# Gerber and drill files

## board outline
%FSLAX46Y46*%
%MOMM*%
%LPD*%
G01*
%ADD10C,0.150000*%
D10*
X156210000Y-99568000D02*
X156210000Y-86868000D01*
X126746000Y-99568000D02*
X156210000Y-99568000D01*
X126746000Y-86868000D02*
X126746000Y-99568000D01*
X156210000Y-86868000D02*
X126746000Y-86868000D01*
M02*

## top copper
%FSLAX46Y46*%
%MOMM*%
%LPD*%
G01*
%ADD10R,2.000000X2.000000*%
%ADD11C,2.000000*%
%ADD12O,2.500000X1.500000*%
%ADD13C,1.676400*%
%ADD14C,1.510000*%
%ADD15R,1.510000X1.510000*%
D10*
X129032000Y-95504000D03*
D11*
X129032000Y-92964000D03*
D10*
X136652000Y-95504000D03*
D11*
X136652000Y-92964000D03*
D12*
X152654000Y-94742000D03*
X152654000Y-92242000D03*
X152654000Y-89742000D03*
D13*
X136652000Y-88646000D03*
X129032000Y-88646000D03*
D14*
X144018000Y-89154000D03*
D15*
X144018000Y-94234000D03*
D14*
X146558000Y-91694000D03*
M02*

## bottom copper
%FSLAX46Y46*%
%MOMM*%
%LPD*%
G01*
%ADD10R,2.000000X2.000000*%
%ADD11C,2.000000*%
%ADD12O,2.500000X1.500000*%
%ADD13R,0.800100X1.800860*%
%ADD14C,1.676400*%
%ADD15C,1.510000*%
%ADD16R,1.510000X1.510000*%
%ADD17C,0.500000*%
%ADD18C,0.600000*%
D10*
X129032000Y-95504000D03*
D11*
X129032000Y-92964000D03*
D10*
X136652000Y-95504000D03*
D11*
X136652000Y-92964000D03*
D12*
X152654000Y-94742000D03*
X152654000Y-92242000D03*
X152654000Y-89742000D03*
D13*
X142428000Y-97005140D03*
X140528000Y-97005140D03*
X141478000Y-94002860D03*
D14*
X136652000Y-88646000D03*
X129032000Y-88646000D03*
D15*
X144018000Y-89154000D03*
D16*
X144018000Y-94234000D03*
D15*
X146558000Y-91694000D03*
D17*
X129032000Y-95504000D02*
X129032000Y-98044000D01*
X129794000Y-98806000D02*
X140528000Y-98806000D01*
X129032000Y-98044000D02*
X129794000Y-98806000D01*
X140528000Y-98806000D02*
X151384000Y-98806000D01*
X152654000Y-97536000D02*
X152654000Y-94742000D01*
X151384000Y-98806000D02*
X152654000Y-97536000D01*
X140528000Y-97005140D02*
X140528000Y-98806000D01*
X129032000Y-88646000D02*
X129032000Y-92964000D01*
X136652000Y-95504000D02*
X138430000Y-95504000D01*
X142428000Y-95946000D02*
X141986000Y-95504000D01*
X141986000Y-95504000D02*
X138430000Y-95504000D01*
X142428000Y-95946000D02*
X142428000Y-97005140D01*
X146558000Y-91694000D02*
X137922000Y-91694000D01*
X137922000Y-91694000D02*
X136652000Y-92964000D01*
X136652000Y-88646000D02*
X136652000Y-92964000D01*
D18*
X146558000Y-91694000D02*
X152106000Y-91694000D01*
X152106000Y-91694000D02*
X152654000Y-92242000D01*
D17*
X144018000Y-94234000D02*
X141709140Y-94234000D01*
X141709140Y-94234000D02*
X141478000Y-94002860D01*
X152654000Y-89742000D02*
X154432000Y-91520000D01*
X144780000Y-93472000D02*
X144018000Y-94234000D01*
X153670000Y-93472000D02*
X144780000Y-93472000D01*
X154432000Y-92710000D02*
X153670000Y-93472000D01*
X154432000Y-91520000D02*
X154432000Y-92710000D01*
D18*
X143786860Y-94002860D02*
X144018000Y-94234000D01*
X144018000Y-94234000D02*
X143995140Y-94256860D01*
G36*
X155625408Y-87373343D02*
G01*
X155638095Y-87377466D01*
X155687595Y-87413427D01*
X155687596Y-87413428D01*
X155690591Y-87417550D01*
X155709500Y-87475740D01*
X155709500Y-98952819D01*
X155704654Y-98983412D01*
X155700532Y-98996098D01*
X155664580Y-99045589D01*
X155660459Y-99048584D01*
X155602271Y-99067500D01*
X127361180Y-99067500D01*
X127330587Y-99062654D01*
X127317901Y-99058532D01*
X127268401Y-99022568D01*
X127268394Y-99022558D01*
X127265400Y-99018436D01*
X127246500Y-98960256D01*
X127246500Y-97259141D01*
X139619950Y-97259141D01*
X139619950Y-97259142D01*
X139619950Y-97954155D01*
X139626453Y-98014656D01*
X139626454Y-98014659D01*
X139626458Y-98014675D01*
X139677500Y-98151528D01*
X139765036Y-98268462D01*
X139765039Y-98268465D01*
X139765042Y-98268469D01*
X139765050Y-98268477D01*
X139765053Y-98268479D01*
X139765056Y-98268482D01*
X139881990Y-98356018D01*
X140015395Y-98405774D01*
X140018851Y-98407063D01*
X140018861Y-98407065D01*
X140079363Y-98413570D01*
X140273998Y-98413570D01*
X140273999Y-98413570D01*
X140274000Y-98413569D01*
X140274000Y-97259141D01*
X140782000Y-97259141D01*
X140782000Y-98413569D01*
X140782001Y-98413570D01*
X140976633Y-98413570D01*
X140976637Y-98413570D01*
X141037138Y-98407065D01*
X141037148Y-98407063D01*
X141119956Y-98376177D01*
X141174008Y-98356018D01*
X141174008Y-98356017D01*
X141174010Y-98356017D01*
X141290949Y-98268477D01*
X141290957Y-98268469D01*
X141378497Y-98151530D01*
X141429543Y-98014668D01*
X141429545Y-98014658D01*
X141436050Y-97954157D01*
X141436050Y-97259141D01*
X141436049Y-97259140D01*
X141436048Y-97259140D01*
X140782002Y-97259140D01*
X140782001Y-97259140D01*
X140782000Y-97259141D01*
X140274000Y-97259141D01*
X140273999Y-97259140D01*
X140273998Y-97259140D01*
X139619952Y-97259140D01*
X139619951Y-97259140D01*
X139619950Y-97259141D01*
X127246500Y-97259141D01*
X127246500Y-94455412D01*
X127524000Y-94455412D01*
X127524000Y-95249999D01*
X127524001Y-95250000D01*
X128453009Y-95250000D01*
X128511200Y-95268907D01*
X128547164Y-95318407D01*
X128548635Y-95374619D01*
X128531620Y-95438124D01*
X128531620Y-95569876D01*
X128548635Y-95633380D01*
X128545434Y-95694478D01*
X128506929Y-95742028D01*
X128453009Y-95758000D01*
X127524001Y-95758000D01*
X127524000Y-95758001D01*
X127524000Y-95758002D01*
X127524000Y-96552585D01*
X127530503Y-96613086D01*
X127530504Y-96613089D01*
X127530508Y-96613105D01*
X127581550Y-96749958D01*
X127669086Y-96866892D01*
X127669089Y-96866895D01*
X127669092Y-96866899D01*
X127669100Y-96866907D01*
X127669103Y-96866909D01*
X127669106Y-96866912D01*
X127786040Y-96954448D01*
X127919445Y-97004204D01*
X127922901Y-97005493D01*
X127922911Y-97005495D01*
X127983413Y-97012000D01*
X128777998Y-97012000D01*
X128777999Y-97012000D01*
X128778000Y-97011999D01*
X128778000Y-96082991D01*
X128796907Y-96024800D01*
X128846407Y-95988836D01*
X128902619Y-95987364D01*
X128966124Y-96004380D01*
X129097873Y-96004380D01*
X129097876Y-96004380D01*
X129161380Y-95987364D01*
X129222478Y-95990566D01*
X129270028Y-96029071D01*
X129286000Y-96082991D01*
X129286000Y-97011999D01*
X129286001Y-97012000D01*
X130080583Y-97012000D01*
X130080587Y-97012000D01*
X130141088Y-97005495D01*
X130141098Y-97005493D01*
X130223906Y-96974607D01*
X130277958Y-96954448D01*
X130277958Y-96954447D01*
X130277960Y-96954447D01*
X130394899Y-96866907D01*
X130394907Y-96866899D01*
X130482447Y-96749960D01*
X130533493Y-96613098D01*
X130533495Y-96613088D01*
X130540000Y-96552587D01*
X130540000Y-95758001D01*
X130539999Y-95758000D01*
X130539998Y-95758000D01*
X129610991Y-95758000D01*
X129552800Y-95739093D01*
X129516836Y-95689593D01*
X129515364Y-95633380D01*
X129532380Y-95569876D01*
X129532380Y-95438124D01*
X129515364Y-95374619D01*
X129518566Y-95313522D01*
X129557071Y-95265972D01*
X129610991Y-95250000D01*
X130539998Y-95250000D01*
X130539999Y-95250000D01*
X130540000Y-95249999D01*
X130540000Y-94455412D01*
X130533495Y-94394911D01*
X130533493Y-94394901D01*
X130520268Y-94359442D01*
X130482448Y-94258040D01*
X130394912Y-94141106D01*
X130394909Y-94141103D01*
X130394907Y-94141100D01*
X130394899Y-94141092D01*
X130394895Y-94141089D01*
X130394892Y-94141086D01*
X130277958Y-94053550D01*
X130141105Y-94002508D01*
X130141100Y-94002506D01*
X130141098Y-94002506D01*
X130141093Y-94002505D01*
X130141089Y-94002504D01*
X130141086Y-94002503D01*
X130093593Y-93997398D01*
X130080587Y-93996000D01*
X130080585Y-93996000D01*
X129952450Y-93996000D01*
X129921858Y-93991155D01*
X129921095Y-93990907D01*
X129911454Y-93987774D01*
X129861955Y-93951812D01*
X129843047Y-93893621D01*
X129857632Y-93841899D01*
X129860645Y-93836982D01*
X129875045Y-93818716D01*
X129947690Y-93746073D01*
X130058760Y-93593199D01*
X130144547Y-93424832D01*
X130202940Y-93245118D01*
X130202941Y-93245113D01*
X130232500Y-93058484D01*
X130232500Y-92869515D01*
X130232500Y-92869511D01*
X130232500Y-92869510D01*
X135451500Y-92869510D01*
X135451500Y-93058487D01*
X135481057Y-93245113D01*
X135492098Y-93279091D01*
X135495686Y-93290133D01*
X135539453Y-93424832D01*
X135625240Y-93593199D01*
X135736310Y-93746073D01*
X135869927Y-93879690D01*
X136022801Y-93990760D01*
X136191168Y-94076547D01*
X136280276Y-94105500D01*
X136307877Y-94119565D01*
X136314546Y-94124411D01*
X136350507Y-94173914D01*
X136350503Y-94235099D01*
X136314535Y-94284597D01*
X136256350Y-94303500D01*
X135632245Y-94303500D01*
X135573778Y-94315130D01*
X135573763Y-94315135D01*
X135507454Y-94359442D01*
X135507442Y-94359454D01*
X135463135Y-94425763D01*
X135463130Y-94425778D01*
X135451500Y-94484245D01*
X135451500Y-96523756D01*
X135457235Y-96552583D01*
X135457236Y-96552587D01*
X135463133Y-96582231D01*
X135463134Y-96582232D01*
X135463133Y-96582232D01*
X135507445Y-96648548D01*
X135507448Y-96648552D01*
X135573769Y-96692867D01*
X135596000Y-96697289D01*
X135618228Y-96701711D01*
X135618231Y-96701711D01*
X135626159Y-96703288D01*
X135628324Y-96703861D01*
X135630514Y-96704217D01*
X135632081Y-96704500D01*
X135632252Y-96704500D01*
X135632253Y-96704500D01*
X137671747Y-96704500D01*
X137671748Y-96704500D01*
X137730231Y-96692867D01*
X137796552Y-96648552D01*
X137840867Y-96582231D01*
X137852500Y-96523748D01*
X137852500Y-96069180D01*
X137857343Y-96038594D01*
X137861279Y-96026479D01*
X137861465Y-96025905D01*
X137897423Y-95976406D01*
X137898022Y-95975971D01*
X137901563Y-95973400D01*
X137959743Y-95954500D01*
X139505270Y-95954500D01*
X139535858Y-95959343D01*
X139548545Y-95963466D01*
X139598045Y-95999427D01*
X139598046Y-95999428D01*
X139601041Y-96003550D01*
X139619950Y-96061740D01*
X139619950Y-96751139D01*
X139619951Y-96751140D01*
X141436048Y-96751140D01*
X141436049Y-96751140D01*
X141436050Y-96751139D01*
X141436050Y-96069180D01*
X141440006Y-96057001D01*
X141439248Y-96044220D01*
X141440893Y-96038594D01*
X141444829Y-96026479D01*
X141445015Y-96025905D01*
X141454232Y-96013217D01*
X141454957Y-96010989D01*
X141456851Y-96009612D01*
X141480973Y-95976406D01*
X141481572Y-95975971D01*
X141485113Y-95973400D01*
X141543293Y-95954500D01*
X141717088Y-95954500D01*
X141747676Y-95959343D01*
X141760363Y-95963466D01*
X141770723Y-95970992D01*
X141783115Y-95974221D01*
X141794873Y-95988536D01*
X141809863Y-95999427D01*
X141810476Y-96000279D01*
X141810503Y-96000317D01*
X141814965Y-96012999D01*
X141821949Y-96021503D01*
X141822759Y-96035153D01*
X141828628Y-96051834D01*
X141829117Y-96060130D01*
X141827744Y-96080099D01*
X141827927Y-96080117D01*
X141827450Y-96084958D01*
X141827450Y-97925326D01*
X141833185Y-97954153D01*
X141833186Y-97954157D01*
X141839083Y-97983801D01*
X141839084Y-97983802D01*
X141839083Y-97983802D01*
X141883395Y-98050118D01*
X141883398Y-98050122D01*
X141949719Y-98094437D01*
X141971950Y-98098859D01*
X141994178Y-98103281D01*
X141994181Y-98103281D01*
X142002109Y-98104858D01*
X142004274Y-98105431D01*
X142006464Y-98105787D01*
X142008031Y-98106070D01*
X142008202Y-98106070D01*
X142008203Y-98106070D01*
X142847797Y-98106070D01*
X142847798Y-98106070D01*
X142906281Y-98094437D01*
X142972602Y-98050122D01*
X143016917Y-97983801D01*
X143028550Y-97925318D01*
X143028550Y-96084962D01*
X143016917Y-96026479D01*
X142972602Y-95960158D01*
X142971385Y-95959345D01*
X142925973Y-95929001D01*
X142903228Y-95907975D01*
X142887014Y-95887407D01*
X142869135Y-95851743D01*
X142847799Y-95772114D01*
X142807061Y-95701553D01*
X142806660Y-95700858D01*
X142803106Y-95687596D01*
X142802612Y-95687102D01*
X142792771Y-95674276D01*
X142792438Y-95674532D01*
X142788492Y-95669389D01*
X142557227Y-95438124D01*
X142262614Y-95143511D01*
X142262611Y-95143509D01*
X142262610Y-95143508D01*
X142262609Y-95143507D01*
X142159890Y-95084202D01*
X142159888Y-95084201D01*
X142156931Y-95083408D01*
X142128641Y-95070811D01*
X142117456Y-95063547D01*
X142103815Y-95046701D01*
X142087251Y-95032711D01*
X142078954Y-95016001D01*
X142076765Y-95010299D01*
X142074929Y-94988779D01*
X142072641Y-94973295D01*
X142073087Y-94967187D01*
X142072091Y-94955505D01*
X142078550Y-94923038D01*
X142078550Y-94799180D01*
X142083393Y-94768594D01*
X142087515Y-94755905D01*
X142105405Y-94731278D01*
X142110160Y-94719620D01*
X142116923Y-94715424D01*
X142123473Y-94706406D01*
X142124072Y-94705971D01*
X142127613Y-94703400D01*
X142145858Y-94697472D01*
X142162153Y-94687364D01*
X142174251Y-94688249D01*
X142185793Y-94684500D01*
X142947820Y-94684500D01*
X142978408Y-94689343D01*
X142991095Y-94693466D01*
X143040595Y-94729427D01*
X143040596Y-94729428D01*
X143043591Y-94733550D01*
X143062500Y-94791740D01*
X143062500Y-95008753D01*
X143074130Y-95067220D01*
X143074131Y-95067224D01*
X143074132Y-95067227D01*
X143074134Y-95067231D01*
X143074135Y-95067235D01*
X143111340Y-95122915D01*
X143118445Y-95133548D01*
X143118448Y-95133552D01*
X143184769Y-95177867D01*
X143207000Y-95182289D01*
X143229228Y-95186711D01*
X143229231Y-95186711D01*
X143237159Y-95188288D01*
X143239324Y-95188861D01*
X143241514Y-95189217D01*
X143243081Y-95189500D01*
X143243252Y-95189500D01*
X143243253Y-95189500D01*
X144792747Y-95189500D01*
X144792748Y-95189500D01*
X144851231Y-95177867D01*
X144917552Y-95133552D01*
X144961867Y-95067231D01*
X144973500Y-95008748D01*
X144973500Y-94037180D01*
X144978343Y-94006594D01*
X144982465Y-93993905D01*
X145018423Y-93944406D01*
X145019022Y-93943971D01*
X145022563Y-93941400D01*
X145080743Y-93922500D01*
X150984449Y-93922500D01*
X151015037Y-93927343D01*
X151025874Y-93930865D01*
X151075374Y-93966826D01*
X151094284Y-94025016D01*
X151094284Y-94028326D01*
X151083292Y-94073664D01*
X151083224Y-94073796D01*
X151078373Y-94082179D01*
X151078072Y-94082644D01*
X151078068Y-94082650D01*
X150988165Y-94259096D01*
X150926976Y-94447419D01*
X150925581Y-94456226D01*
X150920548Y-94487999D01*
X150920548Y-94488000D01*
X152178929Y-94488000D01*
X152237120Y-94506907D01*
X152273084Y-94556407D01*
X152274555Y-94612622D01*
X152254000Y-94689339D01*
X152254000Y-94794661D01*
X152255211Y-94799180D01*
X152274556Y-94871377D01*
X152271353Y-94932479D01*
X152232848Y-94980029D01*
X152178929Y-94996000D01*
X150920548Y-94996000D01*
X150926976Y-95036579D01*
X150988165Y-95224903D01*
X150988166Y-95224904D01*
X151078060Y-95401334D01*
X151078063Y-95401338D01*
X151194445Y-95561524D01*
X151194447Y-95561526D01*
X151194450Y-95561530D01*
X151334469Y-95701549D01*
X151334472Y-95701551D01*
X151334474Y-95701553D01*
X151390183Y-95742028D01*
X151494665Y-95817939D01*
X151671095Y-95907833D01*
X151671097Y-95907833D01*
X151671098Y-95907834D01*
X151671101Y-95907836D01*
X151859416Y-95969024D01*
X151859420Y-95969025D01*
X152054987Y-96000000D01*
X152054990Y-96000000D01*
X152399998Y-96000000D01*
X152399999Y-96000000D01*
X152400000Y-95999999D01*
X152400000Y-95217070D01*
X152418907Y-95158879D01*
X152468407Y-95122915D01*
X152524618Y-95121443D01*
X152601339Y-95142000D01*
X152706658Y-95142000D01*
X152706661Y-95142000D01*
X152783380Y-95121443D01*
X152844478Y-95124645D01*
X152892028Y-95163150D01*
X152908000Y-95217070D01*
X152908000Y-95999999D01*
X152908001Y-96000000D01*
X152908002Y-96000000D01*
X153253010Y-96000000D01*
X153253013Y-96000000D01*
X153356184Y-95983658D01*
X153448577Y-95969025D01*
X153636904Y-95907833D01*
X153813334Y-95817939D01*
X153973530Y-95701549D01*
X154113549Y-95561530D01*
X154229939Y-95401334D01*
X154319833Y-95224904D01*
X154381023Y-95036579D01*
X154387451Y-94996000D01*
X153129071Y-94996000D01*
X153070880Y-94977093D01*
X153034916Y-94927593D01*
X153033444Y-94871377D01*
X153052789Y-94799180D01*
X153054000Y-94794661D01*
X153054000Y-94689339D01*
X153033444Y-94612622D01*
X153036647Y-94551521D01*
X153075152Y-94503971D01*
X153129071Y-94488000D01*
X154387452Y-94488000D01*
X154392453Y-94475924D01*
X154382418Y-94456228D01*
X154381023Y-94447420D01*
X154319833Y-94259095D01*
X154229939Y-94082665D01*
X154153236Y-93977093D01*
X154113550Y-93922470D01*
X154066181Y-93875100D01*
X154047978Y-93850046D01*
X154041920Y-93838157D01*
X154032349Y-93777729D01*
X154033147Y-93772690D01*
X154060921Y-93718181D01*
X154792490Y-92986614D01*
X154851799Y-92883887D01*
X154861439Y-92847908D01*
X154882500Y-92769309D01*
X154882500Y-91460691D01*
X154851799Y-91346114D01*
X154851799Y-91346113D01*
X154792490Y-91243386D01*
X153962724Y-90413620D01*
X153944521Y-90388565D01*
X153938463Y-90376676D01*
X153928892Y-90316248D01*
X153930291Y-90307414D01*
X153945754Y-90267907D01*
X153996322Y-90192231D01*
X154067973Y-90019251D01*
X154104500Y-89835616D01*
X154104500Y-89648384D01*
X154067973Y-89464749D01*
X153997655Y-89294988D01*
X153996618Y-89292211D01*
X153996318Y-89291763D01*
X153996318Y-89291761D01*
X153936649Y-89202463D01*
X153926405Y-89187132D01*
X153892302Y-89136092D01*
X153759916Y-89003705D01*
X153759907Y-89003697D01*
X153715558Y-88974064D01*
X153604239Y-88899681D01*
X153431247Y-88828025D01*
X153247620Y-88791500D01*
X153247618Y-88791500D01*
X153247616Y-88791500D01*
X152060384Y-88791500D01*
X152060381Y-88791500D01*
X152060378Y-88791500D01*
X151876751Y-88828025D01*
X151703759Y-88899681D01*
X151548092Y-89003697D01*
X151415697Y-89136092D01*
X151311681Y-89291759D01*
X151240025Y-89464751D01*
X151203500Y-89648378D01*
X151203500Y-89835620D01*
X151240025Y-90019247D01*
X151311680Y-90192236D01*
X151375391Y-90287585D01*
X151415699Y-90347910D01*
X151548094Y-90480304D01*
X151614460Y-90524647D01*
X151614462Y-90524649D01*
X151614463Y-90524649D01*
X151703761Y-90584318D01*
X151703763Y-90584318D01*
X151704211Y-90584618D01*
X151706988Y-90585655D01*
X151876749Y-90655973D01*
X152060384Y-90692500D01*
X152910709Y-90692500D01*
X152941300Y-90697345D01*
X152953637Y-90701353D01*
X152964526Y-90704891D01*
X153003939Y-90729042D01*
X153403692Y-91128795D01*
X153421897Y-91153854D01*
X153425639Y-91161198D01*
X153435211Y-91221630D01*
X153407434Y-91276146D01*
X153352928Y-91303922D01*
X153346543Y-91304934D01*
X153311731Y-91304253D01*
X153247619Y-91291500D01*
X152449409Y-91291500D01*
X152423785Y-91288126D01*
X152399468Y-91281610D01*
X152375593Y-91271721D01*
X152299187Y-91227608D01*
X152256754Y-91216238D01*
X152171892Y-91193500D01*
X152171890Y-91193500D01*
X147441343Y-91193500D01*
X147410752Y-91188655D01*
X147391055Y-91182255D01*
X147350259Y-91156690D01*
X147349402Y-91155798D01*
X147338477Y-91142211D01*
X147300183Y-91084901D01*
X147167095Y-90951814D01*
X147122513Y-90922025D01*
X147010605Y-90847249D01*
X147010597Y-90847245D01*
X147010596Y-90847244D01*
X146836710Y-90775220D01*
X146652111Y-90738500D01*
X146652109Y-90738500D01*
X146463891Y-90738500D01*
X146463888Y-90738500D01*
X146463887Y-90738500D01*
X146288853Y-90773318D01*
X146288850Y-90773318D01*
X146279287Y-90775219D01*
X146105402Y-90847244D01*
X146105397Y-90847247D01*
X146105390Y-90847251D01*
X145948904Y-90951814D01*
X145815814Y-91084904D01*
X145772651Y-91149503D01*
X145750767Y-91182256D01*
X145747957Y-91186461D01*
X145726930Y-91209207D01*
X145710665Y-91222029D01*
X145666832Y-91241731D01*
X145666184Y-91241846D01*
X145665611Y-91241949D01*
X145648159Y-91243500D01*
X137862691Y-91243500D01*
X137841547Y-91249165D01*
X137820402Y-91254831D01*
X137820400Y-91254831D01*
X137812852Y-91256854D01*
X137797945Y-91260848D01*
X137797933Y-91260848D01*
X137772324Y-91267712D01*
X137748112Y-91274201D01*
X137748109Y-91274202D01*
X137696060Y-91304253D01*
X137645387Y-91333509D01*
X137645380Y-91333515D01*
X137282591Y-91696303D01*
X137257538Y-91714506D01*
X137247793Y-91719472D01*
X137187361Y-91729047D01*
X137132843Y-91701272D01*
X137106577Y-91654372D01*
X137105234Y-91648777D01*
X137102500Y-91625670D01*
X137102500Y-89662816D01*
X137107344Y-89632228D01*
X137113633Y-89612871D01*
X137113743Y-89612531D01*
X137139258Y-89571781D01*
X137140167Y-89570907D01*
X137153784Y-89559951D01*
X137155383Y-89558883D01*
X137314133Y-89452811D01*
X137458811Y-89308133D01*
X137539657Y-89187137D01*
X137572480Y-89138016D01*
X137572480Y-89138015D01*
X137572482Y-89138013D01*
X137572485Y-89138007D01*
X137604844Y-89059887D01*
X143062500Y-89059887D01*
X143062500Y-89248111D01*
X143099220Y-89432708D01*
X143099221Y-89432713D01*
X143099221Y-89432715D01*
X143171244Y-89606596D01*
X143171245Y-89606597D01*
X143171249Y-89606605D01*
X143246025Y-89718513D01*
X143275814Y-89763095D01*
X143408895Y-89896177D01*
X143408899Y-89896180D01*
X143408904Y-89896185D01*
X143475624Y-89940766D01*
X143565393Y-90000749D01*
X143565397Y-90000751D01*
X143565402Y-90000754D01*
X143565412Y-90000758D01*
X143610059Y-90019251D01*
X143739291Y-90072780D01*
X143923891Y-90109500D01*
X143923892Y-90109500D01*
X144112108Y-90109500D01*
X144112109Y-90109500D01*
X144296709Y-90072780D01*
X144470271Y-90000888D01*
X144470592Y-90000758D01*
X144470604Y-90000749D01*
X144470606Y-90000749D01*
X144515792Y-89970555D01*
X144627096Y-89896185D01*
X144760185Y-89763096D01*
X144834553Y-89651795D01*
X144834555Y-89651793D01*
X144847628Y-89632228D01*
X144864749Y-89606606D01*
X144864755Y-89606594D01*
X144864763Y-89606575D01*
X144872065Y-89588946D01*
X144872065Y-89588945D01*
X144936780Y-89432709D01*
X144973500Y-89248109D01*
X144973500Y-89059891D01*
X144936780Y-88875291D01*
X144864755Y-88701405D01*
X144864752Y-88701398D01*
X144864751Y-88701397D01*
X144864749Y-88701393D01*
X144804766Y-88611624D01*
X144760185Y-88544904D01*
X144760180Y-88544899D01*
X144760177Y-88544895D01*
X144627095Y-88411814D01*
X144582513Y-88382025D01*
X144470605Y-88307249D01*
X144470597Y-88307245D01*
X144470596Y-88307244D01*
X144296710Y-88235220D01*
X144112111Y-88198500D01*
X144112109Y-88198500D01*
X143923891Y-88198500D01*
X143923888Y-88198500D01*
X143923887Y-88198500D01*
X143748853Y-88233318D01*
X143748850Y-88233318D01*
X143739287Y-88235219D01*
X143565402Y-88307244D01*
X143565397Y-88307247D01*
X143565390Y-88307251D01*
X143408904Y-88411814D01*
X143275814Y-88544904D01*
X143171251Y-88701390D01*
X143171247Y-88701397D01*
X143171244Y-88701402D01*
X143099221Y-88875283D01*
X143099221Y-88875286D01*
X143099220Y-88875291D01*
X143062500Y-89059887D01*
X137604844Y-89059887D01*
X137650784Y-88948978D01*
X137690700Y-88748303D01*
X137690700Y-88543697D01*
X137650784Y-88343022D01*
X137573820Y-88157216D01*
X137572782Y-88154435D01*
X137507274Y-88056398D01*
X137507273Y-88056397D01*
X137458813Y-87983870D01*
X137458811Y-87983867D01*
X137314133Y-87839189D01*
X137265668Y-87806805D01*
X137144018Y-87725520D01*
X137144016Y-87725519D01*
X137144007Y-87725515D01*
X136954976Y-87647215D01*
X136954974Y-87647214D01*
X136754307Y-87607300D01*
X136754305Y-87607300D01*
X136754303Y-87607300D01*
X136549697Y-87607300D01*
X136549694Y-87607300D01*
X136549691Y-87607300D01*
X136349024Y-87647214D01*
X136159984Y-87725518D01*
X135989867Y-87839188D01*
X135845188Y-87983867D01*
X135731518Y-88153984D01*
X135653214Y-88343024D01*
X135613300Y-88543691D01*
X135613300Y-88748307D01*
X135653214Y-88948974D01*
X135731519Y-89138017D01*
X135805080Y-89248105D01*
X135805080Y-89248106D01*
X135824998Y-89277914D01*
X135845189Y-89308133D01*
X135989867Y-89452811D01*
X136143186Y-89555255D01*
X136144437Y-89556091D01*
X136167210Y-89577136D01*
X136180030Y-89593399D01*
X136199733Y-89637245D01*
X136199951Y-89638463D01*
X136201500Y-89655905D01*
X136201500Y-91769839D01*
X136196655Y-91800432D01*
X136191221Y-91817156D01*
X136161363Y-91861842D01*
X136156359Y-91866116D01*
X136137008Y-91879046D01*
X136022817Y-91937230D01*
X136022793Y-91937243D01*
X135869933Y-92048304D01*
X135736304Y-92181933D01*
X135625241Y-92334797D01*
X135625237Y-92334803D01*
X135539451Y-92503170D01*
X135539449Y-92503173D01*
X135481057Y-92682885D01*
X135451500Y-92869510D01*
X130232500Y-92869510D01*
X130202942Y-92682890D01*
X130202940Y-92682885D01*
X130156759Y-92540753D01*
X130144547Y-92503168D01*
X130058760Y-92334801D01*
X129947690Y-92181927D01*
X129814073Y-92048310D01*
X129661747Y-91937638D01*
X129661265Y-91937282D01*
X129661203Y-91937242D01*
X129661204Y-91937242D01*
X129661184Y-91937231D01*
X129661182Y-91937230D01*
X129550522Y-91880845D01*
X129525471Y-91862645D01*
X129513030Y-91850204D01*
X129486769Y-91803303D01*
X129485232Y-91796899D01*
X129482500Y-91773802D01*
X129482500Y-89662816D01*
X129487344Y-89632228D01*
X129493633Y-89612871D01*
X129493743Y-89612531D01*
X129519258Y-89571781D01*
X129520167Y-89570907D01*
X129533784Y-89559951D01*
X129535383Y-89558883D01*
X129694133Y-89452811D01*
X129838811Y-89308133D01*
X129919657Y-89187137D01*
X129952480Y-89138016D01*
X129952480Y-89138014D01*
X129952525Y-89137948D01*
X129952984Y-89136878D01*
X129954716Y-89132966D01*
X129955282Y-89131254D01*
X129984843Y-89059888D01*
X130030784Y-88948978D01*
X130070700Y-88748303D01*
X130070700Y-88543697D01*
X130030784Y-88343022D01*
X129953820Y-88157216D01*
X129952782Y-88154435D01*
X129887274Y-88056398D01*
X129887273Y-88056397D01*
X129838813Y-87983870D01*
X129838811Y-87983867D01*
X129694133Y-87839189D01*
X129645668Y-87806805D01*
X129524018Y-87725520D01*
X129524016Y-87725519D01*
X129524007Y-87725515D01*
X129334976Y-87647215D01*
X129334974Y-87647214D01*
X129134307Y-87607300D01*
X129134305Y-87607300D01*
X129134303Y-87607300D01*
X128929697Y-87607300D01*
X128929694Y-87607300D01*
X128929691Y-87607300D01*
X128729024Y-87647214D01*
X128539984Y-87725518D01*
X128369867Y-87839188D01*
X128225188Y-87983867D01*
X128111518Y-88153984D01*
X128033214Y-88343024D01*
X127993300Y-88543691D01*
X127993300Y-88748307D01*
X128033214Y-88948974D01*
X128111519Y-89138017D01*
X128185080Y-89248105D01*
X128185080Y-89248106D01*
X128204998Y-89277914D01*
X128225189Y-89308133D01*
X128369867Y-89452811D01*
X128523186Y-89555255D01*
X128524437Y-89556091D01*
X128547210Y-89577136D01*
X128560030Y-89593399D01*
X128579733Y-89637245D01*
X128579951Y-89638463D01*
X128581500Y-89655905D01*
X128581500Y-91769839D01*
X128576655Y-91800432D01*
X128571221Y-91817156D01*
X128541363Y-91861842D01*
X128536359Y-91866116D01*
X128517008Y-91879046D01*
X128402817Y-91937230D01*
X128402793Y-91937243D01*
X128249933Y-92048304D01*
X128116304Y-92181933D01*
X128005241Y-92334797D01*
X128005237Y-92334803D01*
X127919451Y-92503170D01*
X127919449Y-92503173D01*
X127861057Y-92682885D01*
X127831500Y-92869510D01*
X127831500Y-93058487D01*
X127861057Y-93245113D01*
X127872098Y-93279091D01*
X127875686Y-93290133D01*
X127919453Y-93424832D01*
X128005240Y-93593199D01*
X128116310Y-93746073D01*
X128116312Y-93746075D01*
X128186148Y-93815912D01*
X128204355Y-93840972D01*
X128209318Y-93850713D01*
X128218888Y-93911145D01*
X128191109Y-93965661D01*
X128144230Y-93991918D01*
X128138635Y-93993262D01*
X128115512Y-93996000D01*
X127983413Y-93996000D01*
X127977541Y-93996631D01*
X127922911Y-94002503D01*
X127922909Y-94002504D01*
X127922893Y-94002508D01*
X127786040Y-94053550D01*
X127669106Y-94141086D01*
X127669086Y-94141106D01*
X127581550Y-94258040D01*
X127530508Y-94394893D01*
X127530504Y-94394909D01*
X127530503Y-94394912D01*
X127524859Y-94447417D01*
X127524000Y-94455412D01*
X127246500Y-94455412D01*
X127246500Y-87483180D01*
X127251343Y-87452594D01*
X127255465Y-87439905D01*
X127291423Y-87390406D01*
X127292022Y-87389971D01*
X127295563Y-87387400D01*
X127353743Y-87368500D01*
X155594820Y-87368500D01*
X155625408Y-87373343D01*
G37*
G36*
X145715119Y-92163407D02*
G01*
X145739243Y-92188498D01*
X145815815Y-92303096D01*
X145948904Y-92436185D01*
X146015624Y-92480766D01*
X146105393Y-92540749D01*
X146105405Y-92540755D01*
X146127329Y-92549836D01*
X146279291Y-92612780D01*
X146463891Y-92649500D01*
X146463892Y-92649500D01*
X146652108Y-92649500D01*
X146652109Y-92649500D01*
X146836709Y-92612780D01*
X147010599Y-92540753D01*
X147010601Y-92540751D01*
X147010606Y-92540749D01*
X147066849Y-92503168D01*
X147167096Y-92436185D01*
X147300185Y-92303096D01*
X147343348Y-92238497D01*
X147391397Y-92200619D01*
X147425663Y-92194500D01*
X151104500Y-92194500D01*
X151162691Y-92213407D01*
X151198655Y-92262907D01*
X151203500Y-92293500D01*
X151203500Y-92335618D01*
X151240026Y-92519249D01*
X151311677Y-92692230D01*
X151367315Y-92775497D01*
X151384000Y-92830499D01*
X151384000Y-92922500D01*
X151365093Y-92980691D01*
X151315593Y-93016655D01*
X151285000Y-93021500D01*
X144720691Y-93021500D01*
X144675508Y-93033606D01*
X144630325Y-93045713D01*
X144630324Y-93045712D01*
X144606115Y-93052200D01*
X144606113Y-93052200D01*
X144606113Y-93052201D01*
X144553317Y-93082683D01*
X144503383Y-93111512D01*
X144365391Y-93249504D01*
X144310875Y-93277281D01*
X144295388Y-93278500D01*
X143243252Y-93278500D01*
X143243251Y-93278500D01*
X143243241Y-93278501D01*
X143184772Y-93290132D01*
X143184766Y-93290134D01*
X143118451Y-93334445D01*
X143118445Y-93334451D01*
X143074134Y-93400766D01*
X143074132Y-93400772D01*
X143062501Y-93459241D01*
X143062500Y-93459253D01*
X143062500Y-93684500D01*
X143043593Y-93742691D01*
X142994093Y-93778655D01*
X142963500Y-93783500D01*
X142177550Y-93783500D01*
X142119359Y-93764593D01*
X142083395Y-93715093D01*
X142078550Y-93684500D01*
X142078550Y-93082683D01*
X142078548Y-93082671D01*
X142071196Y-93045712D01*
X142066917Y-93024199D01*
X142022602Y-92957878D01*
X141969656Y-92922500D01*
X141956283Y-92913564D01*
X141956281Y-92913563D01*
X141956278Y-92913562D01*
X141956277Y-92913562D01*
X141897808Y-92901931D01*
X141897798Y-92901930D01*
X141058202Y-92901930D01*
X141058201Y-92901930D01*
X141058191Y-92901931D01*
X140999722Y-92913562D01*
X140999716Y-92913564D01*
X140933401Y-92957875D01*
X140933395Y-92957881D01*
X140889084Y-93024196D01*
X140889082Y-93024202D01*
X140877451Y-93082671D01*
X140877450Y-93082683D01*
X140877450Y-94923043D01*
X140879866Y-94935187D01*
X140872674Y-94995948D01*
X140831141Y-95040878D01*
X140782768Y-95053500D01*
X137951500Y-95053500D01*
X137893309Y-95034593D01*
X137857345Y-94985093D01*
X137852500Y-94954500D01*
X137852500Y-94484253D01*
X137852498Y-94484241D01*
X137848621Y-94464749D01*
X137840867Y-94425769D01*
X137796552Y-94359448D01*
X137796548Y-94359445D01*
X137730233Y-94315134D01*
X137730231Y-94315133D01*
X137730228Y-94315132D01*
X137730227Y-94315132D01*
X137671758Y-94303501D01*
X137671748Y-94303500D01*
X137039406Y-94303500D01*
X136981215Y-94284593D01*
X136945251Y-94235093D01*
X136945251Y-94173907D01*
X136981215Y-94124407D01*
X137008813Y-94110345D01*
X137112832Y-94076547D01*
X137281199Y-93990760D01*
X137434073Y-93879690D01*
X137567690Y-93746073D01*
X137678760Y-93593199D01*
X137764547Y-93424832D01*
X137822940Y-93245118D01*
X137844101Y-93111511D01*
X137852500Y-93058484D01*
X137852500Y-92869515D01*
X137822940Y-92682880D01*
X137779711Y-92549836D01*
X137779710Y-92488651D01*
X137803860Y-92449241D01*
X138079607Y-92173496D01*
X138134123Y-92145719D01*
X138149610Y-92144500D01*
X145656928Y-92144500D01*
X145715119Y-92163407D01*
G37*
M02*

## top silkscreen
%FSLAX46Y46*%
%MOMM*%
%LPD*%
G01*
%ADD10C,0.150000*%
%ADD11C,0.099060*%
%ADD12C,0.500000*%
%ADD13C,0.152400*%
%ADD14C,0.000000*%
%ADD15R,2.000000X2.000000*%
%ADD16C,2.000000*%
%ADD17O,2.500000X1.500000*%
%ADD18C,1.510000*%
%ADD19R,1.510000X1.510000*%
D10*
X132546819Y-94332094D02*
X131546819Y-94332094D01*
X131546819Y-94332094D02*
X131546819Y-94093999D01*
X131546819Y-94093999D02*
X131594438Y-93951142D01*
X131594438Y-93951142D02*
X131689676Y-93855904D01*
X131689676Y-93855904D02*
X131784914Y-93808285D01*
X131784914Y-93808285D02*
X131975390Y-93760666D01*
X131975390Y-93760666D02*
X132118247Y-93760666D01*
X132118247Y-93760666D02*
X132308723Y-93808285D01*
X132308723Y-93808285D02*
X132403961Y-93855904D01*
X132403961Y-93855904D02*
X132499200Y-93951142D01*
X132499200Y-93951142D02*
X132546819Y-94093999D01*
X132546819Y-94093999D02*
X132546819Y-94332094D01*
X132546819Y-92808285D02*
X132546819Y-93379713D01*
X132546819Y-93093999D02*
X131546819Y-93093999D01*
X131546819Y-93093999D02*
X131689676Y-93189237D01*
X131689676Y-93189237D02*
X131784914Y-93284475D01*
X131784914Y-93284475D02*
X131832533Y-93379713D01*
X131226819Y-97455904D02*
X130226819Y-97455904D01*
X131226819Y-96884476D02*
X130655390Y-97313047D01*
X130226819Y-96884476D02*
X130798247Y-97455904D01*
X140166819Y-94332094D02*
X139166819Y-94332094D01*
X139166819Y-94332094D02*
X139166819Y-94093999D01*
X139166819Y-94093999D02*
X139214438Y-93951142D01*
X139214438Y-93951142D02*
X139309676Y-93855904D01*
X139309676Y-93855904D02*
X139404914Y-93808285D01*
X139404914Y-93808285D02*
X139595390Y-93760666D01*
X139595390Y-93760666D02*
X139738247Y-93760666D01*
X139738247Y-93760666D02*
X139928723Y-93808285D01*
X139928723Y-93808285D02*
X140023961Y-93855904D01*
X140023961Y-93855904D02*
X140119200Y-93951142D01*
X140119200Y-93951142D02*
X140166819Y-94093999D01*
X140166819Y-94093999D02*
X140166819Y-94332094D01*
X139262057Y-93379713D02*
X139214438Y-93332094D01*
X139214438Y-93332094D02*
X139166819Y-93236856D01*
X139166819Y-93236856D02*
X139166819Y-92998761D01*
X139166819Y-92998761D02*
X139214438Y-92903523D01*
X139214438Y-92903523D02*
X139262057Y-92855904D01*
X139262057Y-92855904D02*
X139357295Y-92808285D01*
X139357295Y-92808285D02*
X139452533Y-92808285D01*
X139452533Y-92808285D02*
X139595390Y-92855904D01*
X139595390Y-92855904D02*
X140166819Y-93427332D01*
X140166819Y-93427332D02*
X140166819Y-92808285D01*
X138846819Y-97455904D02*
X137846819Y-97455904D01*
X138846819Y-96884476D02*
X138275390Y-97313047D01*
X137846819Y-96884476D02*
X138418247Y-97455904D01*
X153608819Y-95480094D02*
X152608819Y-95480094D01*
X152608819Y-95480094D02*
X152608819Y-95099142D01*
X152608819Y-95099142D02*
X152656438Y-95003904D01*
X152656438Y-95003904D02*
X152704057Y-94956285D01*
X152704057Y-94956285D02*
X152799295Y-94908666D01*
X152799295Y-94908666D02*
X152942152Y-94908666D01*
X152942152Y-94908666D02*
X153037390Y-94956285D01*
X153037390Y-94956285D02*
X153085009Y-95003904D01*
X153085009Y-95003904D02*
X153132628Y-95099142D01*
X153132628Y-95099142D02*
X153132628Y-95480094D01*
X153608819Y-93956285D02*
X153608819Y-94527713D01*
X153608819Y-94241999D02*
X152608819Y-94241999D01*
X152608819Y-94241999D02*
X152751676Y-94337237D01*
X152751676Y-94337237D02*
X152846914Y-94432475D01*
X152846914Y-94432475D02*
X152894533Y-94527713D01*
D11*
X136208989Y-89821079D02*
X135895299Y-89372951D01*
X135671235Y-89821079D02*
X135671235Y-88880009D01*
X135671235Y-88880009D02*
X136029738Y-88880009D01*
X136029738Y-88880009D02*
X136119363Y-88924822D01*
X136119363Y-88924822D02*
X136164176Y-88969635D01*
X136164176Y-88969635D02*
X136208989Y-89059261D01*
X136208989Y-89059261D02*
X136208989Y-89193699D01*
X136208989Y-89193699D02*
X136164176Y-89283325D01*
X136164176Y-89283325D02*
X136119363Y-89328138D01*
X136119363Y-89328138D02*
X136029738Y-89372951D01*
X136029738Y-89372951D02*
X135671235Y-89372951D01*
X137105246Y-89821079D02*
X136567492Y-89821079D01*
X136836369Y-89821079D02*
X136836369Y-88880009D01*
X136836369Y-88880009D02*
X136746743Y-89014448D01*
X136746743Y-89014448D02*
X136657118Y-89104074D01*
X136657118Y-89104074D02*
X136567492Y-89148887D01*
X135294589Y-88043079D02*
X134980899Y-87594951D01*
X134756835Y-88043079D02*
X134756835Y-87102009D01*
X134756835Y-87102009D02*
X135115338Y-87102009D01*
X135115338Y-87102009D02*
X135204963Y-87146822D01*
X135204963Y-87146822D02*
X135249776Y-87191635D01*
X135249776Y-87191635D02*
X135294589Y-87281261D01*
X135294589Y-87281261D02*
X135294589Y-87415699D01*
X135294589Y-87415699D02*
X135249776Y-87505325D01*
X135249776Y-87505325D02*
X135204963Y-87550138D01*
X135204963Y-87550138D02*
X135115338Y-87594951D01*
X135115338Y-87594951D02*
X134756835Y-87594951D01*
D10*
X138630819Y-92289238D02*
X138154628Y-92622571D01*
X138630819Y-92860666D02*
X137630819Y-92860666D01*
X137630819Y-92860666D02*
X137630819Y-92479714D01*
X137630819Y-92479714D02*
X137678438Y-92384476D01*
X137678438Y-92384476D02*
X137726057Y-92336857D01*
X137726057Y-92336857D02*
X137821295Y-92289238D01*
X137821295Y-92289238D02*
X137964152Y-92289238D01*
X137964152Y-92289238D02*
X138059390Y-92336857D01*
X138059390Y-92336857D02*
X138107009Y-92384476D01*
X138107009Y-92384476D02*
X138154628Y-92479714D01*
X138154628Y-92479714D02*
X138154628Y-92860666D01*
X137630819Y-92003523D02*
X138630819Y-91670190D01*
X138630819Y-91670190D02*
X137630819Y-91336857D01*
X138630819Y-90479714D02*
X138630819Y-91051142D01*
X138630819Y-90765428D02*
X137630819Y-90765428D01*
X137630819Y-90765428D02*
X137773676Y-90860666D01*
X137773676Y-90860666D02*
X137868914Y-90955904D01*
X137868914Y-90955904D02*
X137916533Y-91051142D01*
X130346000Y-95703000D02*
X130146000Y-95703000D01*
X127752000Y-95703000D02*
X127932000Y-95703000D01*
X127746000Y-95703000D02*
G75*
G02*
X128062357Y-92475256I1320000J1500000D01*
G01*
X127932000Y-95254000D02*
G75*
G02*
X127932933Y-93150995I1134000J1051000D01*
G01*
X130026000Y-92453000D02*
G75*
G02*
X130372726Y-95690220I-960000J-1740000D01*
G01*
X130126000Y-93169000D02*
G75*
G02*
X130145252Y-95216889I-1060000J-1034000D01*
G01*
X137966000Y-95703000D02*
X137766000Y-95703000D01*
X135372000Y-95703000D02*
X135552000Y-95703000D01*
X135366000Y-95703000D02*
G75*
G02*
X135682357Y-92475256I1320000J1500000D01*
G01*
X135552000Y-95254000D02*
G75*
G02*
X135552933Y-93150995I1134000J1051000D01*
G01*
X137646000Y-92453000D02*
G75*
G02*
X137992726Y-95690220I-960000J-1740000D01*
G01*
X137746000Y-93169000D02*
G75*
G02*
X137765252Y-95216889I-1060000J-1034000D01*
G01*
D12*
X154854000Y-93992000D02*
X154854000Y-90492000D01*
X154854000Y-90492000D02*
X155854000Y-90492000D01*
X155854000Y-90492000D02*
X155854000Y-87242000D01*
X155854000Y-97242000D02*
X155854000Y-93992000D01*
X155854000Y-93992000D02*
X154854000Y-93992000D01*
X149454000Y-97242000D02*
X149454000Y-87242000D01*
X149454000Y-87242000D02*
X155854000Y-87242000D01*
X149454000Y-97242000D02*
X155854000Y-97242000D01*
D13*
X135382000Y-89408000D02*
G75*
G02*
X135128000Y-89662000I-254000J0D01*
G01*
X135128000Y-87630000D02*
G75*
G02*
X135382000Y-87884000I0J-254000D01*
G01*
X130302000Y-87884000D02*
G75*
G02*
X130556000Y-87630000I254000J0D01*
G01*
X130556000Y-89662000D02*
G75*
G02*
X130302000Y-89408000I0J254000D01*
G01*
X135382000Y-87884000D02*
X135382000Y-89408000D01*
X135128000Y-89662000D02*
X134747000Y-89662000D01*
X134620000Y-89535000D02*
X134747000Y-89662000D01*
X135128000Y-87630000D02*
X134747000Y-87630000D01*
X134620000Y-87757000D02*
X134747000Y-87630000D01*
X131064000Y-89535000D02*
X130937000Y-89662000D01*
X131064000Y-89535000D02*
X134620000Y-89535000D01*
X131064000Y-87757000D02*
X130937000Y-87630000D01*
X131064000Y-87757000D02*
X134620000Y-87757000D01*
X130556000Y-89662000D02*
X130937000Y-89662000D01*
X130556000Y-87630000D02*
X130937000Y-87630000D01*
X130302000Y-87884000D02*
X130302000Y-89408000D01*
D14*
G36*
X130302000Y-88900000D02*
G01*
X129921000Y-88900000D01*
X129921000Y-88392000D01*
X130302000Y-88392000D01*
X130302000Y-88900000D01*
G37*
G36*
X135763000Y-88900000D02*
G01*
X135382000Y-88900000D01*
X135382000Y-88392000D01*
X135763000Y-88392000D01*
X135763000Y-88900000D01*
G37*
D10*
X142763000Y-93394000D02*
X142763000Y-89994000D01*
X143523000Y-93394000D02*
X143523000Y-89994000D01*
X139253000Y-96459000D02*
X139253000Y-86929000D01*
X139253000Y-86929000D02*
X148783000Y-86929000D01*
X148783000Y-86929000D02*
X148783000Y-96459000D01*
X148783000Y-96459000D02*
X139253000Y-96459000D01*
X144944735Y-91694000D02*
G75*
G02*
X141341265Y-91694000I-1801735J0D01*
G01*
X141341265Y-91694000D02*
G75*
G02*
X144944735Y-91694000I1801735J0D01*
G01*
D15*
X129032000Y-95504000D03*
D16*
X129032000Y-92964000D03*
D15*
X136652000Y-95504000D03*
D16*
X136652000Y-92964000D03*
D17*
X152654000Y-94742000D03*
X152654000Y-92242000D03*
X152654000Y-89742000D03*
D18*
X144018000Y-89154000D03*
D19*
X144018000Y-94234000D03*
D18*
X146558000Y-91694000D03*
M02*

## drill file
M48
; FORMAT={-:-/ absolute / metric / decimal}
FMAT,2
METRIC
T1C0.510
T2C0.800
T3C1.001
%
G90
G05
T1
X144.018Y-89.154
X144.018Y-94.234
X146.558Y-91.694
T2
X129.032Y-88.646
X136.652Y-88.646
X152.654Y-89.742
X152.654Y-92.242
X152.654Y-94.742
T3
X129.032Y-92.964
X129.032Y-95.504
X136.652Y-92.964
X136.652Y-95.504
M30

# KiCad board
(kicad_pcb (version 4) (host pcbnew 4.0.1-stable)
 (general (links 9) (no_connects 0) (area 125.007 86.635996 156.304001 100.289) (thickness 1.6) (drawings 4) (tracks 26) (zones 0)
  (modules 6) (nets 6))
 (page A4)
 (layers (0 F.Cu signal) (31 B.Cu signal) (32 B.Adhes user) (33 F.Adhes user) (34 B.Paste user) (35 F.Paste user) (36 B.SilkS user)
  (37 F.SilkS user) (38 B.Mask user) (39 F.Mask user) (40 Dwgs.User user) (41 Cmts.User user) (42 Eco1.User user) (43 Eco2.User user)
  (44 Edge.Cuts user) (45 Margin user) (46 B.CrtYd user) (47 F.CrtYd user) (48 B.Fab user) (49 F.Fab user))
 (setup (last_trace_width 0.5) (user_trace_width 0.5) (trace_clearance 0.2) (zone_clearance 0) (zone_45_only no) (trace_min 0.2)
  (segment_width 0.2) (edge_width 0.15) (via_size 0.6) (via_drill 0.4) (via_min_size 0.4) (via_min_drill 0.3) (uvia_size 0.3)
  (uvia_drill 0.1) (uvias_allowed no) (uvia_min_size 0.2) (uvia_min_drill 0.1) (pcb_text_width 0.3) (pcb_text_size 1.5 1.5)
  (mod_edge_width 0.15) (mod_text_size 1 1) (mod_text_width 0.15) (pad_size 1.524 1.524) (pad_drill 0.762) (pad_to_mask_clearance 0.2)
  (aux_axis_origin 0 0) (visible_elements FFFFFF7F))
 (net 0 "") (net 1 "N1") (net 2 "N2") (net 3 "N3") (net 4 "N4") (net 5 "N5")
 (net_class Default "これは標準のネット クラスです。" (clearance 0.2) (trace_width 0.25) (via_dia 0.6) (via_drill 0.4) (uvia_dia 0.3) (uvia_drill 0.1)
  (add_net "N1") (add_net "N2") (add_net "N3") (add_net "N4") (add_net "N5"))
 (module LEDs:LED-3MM (layer F.Cu) (at 129.032 95.504 90)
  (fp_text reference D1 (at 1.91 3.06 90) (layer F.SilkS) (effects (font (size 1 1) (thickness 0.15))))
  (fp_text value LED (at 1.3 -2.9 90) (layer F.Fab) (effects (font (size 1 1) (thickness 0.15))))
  (fp_line (start -0.199 1.314) (end -0.199 1.114) (layer F.SilkS) (width 0.15))
  (fp_line (start -0.199 -1.28) (end -0.199 -1.1) (layer F.SilkS) (width 0.15))
  (fp_arc (start 1.301 0.034) (end -0.199 -1.286) (angle 108.5) (layer F.SilkS) (width 0.15))
  (fp_arc (start 1.301 0.034) (end 0.25 -1.1) (angle 85.7) (layer F.SilkS) (width 0.15))
  (fp_arc (start 1.311 0.034) (end 3.051 0.994) (angle 110) (layer F.SilkS) (width 0.15))
  (fp_arc (start 1.301 0.034) (end 2.335 1.094) (angle 87.5) (layer F.SilkS) (width 0.15))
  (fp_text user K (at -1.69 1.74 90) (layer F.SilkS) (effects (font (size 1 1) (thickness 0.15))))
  (pad 1 thru_hole rect (at 0 0 180) (size 2 2) (drill 1.00076) (layers *.Cu *.Mask F.SilkS) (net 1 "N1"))
  (pad 2 thru_hole circle (at 2.54 0 90) (size 2 2) (drill 1.00076) (layers *.Cu *.Mask F.SilkS) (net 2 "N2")))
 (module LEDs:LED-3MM (layer F.Cu) (at 136.652 95.504 90)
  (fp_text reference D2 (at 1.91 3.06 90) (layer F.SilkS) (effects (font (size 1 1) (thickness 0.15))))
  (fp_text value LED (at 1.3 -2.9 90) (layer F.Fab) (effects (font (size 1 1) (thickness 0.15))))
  (fp_line (start -0.199 1.314) (end -0.199 1.114) (layer F.SilkS) (width 0.15))
  (fp_line (start -0.199 -1.28) (end -0.199 -1.1) (layer F.SilkS) (width 0.15))
  (fp_arc (start 1.301 0.034) (end -0.199 -1.286) (angle 108.5) (layer F.SilkS) (width 0.15))
  (fp_arc (start 1.301 0.034) (end 0.25 -1.1) (angle 85.7) (layer F.SilkS) (width 0.15))
  (fp_arc (start 1.311 0.034) (end 3.051 0.994) (angle 110) (layer F.SilkS) (width 0.15))
  (fp_arc (start 1.301 0.034) (end 2.335 1.094) (angle 87.5) (layer F.SilkS) (width 0.15))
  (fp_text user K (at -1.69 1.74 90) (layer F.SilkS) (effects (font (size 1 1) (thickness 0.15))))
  (pad 1 thru_hole rect (at 0 0 180) (size 2 2) (drill 1.00076) (layers *.Cu *.Mask F.SilkS) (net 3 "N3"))
  (pad 2 thru_hole circle (at 2.54 0 90) (size 2 2) (drill 1.00076) (layers *.Cu *.Mask F.SilkS) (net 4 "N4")))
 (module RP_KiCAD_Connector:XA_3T (layer F.Cu) (at 152.654 94.742 90)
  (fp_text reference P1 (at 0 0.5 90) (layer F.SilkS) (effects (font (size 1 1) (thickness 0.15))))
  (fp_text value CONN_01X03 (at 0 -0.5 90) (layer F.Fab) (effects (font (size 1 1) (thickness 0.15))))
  (fp_line (start 0.75 2.2) (end 4.25 2.2) (layer F.SilkS) (width 0.5))
  (fp_line (start 4.25 2.2) (end 4.25 3.2) (layer F.SilkS) (width 0.5))
  (fp_line (start 4.25 3.2) (end 7.5 3.2) (layer F.SilkS) (width 0.5))
  (fp_line (start -2.5 3.2) (end 0.75 3.2) (layer F.SilkS) (width 0.5))
  (fp_line (start 0.75 3.2) (end 0.75 2.2) (layer F.SilkS) (width 0.5))
  (fp_line (start -2.5 -3.2) (end 7.5 -3.2) (layer F.SilkS) (width 0.5))
  (fp_line (start 7.5 -3.2) (end 7.5 3.2) (layer F.SilkS) (width 0.5))
  (fp_line (start -2.5 -3.2) (end -2.5 3.2) (layer F.SilkS) (width 0.5))
  (pad 1 thru_hole oval (at 0 0 90) (size 1.5 2.5) (drill 0.8) (layers *.Cu *.Mask F.SilkS) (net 1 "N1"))
  (pad 2 thru_hole oval (at 2.5 0 90) (size 1.5 2.5) (drill 0.8) (layers *.Cu *.Mask F.SilkS) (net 4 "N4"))
  (pad 3 thru_hole oval (at 5 0 90) (size 1.5 2.5) (drill 0.8) (layers *.Cu *.Mask F.SilkS) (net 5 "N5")))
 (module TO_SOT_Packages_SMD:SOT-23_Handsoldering (layer B.Cu) (at 141.478 95.504 180)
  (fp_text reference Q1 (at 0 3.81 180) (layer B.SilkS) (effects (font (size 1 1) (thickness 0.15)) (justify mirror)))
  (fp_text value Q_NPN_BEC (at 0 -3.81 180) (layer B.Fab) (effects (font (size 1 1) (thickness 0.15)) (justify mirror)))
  (pad 1 smd rect (at -0.95 -1.50114 180) (size 0.8001 1.80086) (layers B.Cu B.Paste B.Mask) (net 3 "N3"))
  (pad 2 smd rect (at 0.95 -1.50114 180) (size 0.8001 1.80086) (layers B.Cu B.Paste B.Mask) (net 1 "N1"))
  (pad 3 smd rect (at 0 1.50114 180) (size 0.8001 1.80086) (layers B.Cu B.Paste B.Mask) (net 5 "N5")))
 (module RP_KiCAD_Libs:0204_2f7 (layer F.Cu) (at 132.842 88.646 180)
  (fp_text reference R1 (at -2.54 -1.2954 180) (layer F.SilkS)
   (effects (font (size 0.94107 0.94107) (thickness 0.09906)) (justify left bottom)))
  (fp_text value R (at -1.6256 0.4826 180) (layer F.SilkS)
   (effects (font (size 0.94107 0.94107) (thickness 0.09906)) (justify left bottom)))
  (fp_arc (start -2.286 -0.762) (end -2.54 -0.762) (angle 90) (layer F.SilkS) (width 0.1524))
  (fp_arc (start -2.286 0.762) (end -2.54 0.762) (angle -90) (layer F.SilkS) (width 0.1524))
  (fp_arc (start 2.286 0.762) (end 2.286 1.016) (angle -90) (layer F.SilkS) (width 0.1524))
  (fp_arc (start 2.286 -0.762) (end 2.286 -1.016) (angle 90) (layer F.SilkS) (width 0.1524))
  (fp_line (start -2.54 0.762) (end -2.54 -0.762) (layer F.SilkS) (width 0.1524))
  (fp_line (start -2.286 -1.016) (end -1.905 -1.016) (layer F.SilkS) (width 0.1524))
  (fp_line (start -1.778 -0.889) (end -1.905 -1.016) (layer F.SilkS) (width 0.1524))
  (fp_line (start -2.286 1.016) (end -1.905 1.016) (layer F.SilkS) (width 0.1524))
  (fp_line (start -1.778 0.889) (end -1.905 1.016) (layer F.SilkS) (width 0.1524))
  (fp_line (start 1.778 -0.889) (end 1.905 -1.016) (layer F.SilkS) (width 0.1524))
  (fp_line (start 1.778 -0.889) (end -1.778 -0.889) (layer F.SilkS) (width 0.1524))
  (fp_line (start 1.778 0.889) (end 1.905 1.016) (layer F.SilkS) (width 0.1524))
  (fp_line (start 1.778 0.889) (end -1.778 0.889) (layer F.SilkS) (width 0.1524))
  (fp_line (start 2.286 -1.016) (end 1.905 -1.016) (layer F.SilkS) (width 0.1524))
  (fp_line (start 2.286 1.016) (end 1.905 1.016) (layer F.SilkS) (width 0.1524))
  (fp_line (start 2.54 0.762) (end 2.54 -0.762) (layer F.SilkS) (width 0.1524))
  (fp_poly (pts (xy 2.54 0.254) (xy 2.921 0.254) (xy 2.921 -0.254) (xy 2.54 -0.254)) (layer F.SilkS) (width 0))
  (fp_poly (pts (xy -2.921 0.254) (xy -2.54 0.254) (xy -2.54 -0.254) (xy -2.921 -0.254)) (layer F.SilkS) (width 0))
  (pad 1 thru_hole circle (at -3.81 0 180) (size 1.6764 1.6764) (drill 0.8) (layers *.Cu *.Mask) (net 4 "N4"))
  (pad 2 thru_hole circle (at 3.81 0 180) (size 1.6764 1.6764) (drill 0.8) (layers *.Cu *.Mask) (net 2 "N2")))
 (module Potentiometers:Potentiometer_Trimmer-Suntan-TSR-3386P (layer F.Cu) (at 144.018 94.234 90)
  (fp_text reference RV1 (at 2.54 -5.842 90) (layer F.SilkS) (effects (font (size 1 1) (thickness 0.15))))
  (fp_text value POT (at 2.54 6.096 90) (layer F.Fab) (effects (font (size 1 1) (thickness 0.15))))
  (fp_line (start 0.84 -1.255) (end 4.24 -1.255) (layer F.SilkS) (width 0.15))
  (fp_line (start 0.84 -0.495) (end 4.24 -0.495) (layer F.SilkS) (width 0.15))
  (fp_line (start -2.225 -4.765) (end 7.305 -4.765) (layer F.SilkS) (width 0.15))
  (fp_line (start 7.305 -4.765) (end 7.305 4.765) (layer F.SilkS) (width 0.15))
  (fp_line (start 7.305 4.765) (end -2.225 4.765) (layer F.SilkS) (width 0.15))
  (fp_line (start -2.225 4.765) (end -2.225 -4.765) (layer F.SilkS) (width 0.15))
  (fp_circle (center 2.54 -0.875) (end 4.115 0) (layer F.SilkS) (width 0.15))
  (pad 3 thru_hole circle (at 5.08 0 90) (size 1.51 1.51) (drill 0.51) (layers *.Cu *.Mask F.SilkS))
  (pad 1 thru_hole rect (at 0 0 90) (size 1.51 1.51) (drill 0.51) (layers *.Cu *.Mask F.SilkS) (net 5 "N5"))
  (pad 2 thru_hole circle (at 2.54 2.54 90) (size 1.51 1.51) (drill 0.51) (layers *.Cu *.Mask F.SilkS) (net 4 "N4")))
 (gr_line (start 156.21 99.568) (end 156.21 86.868) (angle 90) (layer Edge.Cuts) (width 0.15))
 (gr_line (start 126.746 99.568) (end 156.21 99.568) (angle 90) (layer Edge.Cuts) (width 0.15))
 (gr_line (start 126.746 86.868) (end 126.746 99.568) (angle 90) (layer Edge.Cuts) (width 0.15))
 (gr_line (start 156.21 86.868) (end 126.746 86.868) (angle 90) (layer Edge.Cuts) (width 0.15))
 (segment (start 129.032 95.504) (end 129.032 98.044) (width 0.5) (layer B.Cu) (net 1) (status 400000))
 (segment (start 129.794 98.806) (end 140.528 98.806) (width 0.5) (layer B.Cu) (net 1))
 (segment (start 129.032 98.044) (end 129.794 98.806) (width 0.5) (layer B.Cu) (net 1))
 (segment (start 140.528 98.806) (end 151.384 98.806) (width 0.5) (layer B.Cu) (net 1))
 (segment (start 152.654 97.536) (end 152.654 94.742) (width 0.5) (layer B.Cu) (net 1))
 (segment (start 151.384 98.806) (end 152.654 97.536) (width 0.5) (layer B.Cu) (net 1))
 (segment (start 140.528 97.00514) (end 140.528 98.806) (width 0.5) (layer B.Cu) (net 1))
 (segment (start 129.032 88.646) (end 129.032 92.964) (width 0.5) (layer B.Cu) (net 2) (status C00000))
 (segment (start 136.652 95.504) (end 138.43 95.504) (width 0.5) (layer B.Cu) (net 3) (status 400000))
 (segment (start 142.428 95.946) (end 141.986 95.504) (width 0.5) (layer B.Cu) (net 3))
 (segment (start 141.986 95.504) (end 138.43 95.504) (width 0.5) (layer B.Cu) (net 3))
 (segment (start 142.428 95.946) (end 142.428 97.00514) (width 0.5) (layer B.Cu) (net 3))
 (segment (start 146.558 91.694) (end 137.922 91.694) (width 0.5) (layer B.Cu) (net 4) (status 400000))
 (segment (start 137.922 91.694) (end 136.652 92.964) (width 0.5) (layer B.Cu) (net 4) (status 800000))
 (segment (start 136.652 88.646) (end 136.652 92.964) (width 0.5) (layer B.Cu) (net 4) (status C00000))
 (segment (start 146.558 91.694) (end 152.106 91.694) (width 0.6) (layer B.Cu) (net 4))
 (segment (start 152.106 91.694) (end 152.654 92.242) (width 0.6) (layer B.Cu) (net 4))
 (segment (start 144.018 94.234) (end 141.70914 94.234) (width 0.5) (layer B.Cu) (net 5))
 (segment (start 141.70914 94.234) (end 141.478 94.00286) (width 0.5) (layer B.Cu) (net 5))
 (segment (start 152.654 89.742) (end 154.432 91.52) (width 0.5) (layer B.Cu) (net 5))
 (segment (start 144.78 93.472) (end 144.018 94.234) (width 0.5) (layer B.Cu) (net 5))
 (segment (start 153.67 93.472) (end 144.78 93.472) (width 0.5) (layer B.Cu) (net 5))
 (segment (start 154.432 92.71) (end 153.67 93.472) (width 0.5) (layer B.Cu) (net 5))
 (segment (start 154.432 91.52) (end 154.432 92.71) (width 0.5) (layer B.Cu) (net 5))
 (segment (start 143.78686 94.00286) (end 144.018 94.234) (width 0.6) (layer B.Cu) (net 5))
 (segment (start 144.018 94.234) (end 143.99514 94.25686) (width 0.6) (layer B.Cu) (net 5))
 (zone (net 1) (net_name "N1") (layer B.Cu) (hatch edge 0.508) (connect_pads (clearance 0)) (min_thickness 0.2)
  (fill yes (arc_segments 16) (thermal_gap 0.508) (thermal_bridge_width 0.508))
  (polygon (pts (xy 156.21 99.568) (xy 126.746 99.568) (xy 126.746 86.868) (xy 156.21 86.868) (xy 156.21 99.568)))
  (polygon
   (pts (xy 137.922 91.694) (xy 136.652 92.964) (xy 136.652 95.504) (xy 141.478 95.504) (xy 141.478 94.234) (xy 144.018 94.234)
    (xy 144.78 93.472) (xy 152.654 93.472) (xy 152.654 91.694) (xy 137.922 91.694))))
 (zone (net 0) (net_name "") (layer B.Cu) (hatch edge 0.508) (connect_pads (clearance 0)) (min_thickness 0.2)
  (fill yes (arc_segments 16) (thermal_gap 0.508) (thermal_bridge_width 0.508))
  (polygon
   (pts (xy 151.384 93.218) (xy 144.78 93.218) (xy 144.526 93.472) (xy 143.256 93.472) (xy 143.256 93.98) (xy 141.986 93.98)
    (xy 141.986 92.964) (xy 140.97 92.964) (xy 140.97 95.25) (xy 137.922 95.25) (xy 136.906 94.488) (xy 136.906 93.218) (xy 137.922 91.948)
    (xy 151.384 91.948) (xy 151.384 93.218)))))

